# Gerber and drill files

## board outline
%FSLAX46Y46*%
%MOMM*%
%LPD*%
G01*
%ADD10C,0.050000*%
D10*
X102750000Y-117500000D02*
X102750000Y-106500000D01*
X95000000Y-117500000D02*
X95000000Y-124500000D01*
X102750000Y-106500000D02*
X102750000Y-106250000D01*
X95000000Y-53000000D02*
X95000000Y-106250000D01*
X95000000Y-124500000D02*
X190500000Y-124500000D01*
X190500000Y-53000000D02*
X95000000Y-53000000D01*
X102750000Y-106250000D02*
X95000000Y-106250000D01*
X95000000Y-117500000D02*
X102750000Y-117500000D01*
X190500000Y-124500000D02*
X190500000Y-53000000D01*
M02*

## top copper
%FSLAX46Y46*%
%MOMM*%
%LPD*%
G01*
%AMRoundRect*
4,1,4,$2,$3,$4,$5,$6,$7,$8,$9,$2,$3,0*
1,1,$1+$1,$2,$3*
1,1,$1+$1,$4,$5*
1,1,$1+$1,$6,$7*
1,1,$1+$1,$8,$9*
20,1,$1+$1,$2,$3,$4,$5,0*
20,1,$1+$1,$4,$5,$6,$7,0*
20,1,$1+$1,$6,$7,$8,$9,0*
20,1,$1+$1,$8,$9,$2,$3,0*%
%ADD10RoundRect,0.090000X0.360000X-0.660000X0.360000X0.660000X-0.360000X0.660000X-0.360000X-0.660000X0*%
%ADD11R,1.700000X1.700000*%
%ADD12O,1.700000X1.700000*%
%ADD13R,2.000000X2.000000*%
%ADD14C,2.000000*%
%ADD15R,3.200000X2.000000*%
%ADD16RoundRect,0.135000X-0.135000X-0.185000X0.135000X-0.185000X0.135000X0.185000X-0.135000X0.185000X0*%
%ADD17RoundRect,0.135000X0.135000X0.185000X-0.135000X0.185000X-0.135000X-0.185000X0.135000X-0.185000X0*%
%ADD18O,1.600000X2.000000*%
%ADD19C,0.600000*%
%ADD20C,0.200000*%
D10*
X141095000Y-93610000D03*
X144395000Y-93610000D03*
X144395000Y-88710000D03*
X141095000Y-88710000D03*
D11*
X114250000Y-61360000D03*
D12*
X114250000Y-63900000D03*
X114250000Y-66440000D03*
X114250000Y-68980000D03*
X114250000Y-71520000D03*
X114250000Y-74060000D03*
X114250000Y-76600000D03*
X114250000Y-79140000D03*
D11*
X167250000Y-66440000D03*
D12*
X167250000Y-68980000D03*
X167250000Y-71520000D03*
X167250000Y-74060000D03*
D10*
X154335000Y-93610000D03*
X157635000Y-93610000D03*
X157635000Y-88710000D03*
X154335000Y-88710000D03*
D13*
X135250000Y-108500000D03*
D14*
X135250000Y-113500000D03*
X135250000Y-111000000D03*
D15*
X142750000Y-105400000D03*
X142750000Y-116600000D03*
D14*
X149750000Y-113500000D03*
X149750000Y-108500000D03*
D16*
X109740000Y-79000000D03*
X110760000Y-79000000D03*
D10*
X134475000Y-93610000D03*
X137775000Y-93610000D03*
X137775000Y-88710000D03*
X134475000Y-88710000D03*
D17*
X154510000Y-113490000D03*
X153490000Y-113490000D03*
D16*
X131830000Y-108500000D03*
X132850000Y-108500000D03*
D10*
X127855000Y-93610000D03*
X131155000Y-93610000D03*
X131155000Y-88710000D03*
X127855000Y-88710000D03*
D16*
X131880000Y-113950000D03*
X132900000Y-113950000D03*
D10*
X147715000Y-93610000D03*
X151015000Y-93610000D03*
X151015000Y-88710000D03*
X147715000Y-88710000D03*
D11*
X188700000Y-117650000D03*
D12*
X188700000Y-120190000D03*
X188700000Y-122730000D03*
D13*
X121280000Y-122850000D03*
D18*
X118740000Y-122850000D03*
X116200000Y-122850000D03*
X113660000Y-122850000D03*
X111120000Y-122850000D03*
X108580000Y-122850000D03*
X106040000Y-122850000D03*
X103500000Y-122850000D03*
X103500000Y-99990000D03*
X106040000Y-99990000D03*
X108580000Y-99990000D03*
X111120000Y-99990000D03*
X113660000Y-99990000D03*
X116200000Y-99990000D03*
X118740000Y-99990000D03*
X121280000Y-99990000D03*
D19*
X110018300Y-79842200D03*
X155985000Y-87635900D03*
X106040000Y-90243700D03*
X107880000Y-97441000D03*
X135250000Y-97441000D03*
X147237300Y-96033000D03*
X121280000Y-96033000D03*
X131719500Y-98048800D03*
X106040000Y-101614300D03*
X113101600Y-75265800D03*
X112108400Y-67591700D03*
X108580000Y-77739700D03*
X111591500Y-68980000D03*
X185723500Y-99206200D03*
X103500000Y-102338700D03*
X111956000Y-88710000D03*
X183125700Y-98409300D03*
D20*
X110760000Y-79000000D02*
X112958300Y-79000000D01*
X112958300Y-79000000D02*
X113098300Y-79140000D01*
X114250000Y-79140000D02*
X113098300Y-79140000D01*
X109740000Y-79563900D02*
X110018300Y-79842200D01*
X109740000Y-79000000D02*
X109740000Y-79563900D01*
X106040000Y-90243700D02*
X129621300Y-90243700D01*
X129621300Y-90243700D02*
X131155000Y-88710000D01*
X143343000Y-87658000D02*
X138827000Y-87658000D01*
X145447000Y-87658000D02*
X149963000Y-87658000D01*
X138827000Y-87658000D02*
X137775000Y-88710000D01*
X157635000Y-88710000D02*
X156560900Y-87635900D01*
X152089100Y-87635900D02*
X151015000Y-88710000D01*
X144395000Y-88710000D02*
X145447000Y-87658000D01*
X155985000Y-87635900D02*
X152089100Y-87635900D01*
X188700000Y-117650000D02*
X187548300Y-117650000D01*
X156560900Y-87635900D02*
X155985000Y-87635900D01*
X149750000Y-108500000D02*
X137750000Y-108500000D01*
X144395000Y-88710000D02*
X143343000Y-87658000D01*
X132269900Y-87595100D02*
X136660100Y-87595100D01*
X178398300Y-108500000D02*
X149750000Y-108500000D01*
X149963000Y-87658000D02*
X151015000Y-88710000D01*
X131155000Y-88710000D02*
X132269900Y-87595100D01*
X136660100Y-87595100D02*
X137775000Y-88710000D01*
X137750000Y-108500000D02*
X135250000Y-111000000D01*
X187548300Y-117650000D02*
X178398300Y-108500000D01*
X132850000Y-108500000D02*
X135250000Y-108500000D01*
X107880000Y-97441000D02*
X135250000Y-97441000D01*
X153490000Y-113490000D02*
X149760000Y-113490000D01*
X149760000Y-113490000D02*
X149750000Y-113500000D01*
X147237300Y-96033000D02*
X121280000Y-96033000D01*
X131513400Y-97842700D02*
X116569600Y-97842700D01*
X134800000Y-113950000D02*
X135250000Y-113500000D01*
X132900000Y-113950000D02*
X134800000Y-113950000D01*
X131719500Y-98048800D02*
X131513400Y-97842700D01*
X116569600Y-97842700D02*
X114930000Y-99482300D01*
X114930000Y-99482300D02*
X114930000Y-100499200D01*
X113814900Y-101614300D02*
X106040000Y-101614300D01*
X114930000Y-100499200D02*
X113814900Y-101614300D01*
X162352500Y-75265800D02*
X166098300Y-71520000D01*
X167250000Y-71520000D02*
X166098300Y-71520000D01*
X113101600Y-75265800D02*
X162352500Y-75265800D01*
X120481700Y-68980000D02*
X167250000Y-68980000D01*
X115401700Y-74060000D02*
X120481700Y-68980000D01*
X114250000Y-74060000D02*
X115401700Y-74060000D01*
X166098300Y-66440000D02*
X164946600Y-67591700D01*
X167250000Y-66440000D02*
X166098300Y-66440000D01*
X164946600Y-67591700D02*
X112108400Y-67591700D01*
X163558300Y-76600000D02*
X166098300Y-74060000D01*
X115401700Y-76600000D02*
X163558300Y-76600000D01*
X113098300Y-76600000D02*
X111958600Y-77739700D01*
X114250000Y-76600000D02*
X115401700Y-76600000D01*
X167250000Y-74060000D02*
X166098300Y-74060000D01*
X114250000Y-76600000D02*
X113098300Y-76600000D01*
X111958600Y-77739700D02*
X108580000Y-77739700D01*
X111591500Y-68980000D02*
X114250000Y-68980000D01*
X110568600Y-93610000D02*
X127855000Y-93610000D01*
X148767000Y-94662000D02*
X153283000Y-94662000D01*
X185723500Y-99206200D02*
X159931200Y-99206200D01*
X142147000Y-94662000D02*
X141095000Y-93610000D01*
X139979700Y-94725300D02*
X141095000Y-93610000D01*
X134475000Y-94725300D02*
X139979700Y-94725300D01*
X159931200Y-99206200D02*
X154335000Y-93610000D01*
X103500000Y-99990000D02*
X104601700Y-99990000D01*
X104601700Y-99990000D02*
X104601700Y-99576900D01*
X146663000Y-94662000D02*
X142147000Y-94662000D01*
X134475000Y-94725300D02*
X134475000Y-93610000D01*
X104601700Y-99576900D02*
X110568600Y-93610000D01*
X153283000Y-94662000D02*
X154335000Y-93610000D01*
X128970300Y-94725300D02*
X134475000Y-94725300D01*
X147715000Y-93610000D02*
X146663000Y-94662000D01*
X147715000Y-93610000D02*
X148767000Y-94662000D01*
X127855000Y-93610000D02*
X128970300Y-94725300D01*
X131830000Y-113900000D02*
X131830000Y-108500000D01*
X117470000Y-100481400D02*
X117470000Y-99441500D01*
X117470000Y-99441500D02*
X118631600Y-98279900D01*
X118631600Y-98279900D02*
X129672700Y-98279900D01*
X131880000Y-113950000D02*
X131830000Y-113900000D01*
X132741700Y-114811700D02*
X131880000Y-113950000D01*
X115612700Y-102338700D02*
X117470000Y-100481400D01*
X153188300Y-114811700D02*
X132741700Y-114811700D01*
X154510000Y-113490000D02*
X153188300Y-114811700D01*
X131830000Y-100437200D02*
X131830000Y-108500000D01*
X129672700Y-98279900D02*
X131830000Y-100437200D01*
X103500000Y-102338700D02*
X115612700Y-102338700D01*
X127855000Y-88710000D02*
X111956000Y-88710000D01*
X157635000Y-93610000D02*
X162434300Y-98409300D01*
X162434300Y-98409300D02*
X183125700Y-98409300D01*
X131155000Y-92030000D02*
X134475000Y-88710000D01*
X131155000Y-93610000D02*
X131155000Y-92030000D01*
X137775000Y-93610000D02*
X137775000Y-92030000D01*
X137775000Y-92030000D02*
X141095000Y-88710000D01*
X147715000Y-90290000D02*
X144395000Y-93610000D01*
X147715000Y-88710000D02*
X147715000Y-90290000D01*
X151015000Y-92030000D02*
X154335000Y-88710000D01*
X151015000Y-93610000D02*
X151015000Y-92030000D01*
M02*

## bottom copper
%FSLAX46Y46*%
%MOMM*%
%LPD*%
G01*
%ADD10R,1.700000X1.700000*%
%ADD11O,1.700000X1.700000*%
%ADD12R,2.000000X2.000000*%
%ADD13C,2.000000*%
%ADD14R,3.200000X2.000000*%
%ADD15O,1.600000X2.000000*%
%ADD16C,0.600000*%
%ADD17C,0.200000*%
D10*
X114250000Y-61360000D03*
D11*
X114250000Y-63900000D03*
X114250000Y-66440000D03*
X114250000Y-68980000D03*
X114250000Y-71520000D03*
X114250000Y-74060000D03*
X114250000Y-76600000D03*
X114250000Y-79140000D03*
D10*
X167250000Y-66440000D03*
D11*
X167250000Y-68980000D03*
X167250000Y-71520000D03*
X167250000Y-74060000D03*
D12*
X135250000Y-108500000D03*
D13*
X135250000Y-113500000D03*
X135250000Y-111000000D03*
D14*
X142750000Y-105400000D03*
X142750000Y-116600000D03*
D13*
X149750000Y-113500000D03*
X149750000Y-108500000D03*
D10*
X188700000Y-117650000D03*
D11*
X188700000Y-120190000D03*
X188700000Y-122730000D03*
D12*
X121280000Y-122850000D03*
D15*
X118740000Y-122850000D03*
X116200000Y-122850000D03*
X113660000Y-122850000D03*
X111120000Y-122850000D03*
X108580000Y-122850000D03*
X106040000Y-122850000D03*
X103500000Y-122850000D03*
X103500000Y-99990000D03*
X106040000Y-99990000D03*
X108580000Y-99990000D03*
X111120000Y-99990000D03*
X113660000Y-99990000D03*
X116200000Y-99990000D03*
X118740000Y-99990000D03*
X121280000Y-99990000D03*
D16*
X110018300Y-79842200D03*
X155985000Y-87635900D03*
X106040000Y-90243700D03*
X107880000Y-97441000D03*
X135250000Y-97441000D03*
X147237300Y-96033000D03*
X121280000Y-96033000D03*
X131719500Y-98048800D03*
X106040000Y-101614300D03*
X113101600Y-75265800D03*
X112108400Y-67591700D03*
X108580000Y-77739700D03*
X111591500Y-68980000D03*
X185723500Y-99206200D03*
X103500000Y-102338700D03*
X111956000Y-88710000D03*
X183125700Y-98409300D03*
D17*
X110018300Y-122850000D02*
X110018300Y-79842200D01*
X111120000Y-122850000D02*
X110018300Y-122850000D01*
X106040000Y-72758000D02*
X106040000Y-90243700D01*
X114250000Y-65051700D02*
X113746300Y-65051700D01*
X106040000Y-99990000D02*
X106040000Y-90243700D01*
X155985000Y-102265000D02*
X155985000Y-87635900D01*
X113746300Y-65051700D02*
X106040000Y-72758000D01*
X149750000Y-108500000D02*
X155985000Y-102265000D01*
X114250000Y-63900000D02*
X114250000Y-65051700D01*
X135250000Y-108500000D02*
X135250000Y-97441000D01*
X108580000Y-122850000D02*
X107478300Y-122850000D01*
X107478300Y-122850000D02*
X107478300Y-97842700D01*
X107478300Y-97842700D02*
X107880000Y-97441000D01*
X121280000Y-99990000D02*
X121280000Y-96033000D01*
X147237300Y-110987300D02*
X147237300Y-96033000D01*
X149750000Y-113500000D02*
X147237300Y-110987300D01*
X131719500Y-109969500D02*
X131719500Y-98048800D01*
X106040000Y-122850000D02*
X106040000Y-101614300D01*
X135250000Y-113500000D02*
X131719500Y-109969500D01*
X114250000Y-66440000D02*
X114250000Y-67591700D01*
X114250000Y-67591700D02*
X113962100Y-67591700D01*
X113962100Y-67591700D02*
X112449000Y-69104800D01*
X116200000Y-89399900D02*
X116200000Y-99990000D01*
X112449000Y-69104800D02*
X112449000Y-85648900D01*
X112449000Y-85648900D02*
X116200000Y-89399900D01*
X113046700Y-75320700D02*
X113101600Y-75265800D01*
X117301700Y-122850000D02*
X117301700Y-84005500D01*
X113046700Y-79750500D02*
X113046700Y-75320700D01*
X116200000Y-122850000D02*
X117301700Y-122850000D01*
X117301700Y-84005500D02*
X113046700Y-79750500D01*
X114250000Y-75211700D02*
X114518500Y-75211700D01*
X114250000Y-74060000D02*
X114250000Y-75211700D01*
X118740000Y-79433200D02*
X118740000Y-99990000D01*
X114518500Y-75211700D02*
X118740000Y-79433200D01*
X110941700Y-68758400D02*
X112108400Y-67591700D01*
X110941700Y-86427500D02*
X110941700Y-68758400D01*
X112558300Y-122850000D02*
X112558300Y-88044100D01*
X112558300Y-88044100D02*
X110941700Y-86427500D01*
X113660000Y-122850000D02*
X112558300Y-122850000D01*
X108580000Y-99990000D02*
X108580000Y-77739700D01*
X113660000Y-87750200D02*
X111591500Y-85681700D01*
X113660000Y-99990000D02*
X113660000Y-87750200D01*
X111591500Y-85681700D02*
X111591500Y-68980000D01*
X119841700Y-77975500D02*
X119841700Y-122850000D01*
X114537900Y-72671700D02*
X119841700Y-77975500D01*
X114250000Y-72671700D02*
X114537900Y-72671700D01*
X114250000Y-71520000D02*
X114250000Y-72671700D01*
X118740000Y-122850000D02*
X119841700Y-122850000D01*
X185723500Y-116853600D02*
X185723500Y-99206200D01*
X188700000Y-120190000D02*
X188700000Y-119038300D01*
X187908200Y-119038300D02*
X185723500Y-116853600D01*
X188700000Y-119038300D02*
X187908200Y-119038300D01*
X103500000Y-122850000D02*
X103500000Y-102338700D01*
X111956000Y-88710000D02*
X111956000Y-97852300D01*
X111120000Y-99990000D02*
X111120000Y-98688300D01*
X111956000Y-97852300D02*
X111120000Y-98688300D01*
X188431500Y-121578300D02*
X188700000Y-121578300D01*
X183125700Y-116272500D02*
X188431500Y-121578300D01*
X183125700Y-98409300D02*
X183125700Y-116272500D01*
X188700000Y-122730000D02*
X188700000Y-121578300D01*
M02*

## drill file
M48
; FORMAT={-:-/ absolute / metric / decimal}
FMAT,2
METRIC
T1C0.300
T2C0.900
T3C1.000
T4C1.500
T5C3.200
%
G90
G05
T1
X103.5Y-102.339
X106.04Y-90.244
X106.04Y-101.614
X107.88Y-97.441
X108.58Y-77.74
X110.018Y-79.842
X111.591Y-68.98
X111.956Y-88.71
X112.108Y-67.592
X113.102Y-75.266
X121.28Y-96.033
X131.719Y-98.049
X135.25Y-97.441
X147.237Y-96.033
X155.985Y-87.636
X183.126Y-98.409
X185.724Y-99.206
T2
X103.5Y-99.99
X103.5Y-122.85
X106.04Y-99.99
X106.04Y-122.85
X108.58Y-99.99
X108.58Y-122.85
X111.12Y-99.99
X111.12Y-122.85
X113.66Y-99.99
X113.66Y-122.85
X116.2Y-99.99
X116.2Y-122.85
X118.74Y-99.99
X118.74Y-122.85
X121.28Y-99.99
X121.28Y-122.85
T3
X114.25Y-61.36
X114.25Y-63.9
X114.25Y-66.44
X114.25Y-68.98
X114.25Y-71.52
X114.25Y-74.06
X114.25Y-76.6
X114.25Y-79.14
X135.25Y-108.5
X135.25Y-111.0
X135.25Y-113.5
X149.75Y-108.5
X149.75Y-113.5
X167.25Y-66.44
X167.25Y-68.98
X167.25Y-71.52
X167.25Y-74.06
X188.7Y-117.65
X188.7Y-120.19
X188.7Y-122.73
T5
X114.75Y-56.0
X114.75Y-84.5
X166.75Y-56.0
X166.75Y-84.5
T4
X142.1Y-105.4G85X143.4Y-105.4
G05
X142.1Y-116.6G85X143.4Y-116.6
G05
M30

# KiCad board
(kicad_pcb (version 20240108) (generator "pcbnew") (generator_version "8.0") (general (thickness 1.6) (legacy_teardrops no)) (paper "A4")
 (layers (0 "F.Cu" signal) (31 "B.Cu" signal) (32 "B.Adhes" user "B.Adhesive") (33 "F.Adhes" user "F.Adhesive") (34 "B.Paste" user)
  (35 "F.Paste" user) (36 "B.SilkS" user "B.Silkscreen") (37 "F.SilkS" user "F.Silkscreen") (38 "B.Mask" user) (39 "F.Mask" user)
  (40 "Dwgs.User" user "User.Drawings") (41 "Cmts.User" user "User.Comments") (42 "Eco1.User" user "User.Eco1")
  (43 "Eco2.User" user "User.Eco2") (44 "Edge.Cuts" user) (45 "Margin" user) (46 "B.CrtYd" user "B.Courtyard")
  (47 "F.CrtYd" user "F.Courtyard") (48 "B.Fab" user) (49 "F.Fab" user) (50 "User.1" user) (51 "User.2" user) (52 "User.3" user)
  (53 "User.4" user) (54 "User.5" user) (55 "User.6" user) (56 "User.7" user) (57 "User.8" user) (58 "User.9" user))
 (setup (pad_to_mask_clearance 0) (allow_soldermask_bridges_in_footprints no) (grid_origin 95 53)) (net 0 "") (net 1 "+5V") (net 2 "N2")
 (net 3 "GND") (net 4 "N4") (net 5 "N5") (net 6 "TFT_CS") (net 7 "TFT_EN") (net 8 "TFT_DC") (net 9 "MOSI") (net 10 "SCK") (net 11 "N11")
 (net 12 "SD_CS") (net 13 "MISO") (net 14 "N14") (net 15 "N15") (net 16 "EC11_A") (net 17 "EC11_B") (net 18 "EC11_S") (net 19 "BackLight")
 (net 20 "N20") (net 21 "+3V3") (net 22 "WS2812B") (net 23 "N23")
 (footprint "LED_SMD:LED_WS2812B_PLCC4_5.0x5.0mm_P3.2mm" (layer "F.Cu") (at 142.745 91.16 90)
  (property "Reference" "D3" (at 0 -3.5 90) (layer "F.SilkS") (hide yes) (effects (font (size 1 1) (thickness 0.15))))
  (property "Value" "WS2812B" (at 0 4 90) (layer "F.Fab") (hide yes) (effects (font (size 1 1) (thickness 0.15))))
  (pad "1" smd roundrect (at -2.45 -1.65 90) (size 1.5 0.9) (layers "F.Cu" "F.Paste" "F.Mask") (roundrect_rratio 0.1) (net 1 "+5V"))
  (pad "2" smd roundrect (at -2.45 1.65 90) (size 1.5 0.9) (layers "F.Cu" "F.Paste" "F.Mask") (roundrect_rratio 0.1) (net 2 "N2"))
  (pad "3" smd roundrect (at 2.45 1.65 90) (size 1.5 0.9) (layers "F.Cu" "F.Paste" "F.Mask") (roundrect_rratio 0.1) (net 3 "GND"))
  (pad "4" smd roundrect (at 2.45 -1.65 90) (size 1.5 0.9) (layers "F.Cu" "F.Paste" "F.Mask") (roundrect_rratio 0.1) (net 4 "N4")))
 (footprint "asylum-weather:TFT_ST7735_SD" (layer "F.Cu") (at 134.25 70)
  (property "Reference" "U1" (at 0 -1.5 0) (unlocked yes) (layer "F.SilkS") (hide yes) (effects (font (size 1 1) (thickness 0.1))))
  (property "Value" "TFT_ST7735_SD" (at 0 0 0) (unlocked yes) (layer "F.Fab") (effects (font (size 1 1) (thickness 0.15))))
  (pad "" np_thru_hole circle (at -19.5 -14) (size 3.2 3.2) (drill 3.2) (layers "*.Cu" "*.Mask"))
  (pad "" np_thru_hole circle (at -19.5 14.5) (size 3.2 3.2) (drill 3.2) (layers "*.Cu" "*.Mask"))
  (pad "" np_thru_hole circle (at 32.5 -14) (size 3.2 3.2) (drill 3.2) (layers "*.Cu" "*.Mask"))
  (pad "" np_thru_hole circle (at 32.5 14.5) (size 3.2 3.2) (drill 3.2) (layers "*.Cu" "*.Mask"))
  (pad "1" thru_hole rect (at -20 -8.64) (size 1.7 1.7) (drill 1) (layers "*.Cu" "*.Mask") (remove_unused_layers no) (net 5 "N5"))
  (pad "2" thru_hole oval (at -20 -6.1) (size 1.7 1.7) (drill 1) (layers "*.Cu" "*.Mask") (remove_unused_layers no) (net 3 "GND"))
  (pad "3" thru_hole oval (at -20 -3.56) (size 1.7 1.7) (drill 1) (layers "*.Cu" "*.Mask") (remove_unused_layers no) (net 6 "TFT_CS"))
  (pad "4" thru_hole oval (at -20 -1.02) (size 1.7 1.7) (drill 1) (layers "*.Cu" "*.Mask") (remove_unused_layers no) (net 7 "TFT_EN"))
  (pad "5" thru_hole oval (at -20 1.52) (size 1.7 1.7) (drill 1) (layers "*.Cu" "*.Mask") (remove_unused_layers no) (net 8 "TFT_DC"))
  (pad "6" thru_hole oval (at -20 4.06) (size 1.7 1.7) (drill 1) (layers "*.Cu" "*.Mask") (remove_unused_layers no) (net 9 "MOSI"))
  (pad "7" thru_hole oval (at -20 6.6) (size 1.7 1.7) (drill 1) (layers "*.Cu" "*.Mask") (remove_unused_layers no) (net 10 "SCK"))
  (pad "8" thru_hole oval (at -20 9.14) (size 1.7 1.7) (drill 1) (layers "*.Cu" "*.Mask") (remove_unused_layers no) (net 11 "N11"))
  (pad "9" thru_hole rect (at 33 -3.56) (size 1.7 1.7) (drill 1) (layers "*.Cu" "*.Mask") (remove_unused_layers no) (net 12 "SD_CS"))
  (pad "10" thru_hole oval (at 33 -1.02) (size 1.7 1.7) (drill 1) (layers "*.Cu" "*.Mask") (remove_unused_layers no) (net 9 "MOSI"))
  (pad "11" thru_hole oval (at 33 1.52) (size 1.7 1.7) (drill 1) (layers "*.Cu" "*.Mask") (remove_unused_layers no) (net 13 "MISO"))
  (pad "12" thru_hole oval (at 33 4.06) (size 1.7 1.7) (drill 1) (layers "*.Cu" "*.Mask") (remove_unused_layers no) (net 10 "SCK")))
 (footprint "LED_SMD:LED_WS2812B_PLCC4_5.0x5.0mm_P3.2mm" (layer "F.Cu") (at 155.985 91.16 90)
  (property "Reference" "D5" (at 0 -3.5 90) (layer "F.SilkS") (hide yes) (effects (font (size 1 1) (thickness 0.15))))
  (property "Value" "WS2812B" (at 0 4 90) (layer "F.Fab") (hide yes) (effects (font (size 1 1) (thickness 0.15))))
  (pad "1" smd roundrect (at -2.45 -1.65 90) (size 1.5 0.9) (layers "F.Cu" "F.Paste" "F.Mask") (roundrect_rratio 0.1) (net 1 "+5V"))
  (pad "2" smd roundrect (at -2.45 1.65 90) (size 1.5 0.9) (layers "F.Cu" "F.Paste" "F.Mask") (roundrect_rratio 0.1) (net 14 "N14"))
  (pad "3" smd roundrect (at 2.45 1.65 90) (size 1.5 0.9) (layers "F.Cu" "F.Paste" "F.Mask") (roundrect_rratio 0.1) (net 3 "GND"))
  (pad "4" smd roundrect (at 2.45 -1.65 90) (size 1.5 0.9) (layers "F.Cu" "F.Paste" "F.Mask") (roundrect_rratio 0.1) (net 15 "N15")))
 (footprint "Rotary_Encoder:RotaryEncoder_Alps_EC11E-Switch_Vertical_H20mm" (layer "F.Cu") (at 135.25 108.5)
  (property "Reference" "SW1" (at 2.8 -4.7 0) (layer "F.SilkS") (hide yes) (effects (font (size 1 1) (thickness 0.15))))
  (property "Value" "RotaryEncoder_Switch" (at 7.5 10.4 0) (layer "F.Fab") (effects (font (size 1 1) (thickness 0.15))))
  (pad "A" thru_hole rect (at 0 0) (size 2 2) (drill 1) (layers "*.Cu" "*.Mask") (remove_unused_layers no) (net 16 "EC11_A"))
  (pad "B" thru_hole circle (at 0 5) (size 2 2) (drill 1) (layers "*.Cu" "*.Mask") (remove_unused_layers no) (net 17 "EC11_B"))
  (pad "C" thru_hole circle (at 0 2.5) (size 2 2) (drill 1) (layers "*.Cu" "*.Mask") (remove_unused_layers no) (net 3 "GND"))
  (pad "MP" thru_hole rect (at 7.5 -3.1) (size 3.2 2) (drill oval 2.8 1.5) (layers "*.Cu" "*.Mask") (remove_unused_layers no))
  (pad "MP" thru_hole rect (at 7.5 8.1) (size 3.2 2) (drill oval 2.8 1.5) (layers "*.Cu" "*.Mask") (remove_unused_layers no))
  (pad "S1" thru_hole circle (at 14.5 5) (size 2 2) (drill 1) (layers "*.Cu" "*.Mask") (remove_unused_layers no) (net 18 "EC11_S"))
  (pad "S2" thru_hole circle (at 14.5 0) (size 2 2) (drill 1) (layers "*.Cu" "*.Mask") (remove_unused_layers no) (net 3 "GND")))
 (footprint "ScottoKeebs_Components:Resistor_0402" (layer "F.Cu") (at 110.25 79)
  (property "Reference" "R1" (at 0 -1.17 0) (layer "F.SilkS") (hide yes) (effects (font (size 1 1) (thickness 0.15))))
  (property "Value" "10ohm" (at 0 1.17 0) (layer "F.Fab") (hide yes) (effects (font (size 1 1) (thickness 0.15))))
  (pad "1" smd roundrect (at -0.51 0) (size 0.54 0.64) (layers "F.Cu" "F.Paste" "F.Mask") (roundrect_rratio 0.25) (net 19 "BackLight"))
  (pad "2" smd roundrect (at 0.51 0) (size 0.54 0.64) (layers "F.Cu" "F.Paste" "F.Mask") (roundrect_rratio 0.25) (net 11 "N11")))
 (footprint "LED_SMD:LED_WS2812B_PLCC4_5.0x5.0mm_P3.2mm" (layer "F.Cu") (at 136.125 91.16 90)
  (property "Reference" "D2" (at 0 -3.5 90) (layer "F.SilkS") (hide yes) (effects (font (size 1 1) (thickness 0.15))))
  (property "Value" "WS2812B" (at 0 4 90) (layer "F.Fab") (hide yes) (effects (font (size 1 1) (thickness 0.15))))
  (pad "1" smd roundrect (at -2.45 -1.65 90) (size 1.5 0.9) (layers "F.Cu" "F.Paste" "F.Mask") (roundrect_rratio 0.1) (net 1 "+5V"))
  (pad "2" smd roundrect (at -2.45 1.65 90) (size 1.5 0.9) (layers "F.Cu" "F.Paste" "F.Mask") (roundrect_rratio 0.1) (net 4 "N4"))
  (pad "3" smd roundrect (at 2.45 1.65 90) (size 1.5 0.9) (layers "F.Cu" "F.Paste" "F.Mask") (roundrect_rratio 0.1) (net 3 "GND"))
  (pad "4" smd roundrect (at 2.45 -1.65 90) (size 1.5 0.9) (layers "F.Cu" "F.Paste" "F.Mask") (roundrect_rratio 0.1) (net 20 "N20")))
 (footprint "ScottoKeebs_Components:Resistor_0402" (layer "F.Cu") (at 154 113.49 180)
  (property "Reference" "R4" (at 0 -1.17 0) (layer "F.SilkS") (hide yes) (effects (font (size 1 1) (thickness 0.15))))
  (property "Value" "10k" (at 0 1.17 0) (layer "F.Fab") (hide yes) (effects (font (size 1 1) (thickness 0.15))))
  (pad "1" smd roundrect (at -0.51 0 180) (size 0.54 0.64) (layers "F.Cu" "F.Paste" "F.Mask") (roundrect_rratio 0.25) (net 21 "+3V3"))
  (pad "2" smd roundrect (at 0.51 0 180) (size 0.54 0.64) (layers "F.Cu" "F.Paste" "F.Mask") (roundrect_rratio 0.25) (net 18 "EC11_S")))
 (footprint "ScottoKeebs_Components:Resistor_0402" (layer "F.Cu") (at 132.34 108.5)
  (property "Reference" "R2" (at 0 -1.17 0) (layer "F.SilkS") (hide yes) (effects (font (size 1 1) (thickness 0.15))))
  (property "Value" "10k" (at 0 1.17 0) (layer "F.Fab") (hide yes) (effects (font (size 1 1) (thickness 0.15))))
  (pad "1" smd roundrect (at -0.51 0) (size 0.54 0.64) (layers "F.Cu" "F.Paste" "F.Mask") (roundrect_rratio 0.25) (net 21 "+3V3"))
  (pad "2" smd roundrect (at 0.51 0) (size 0.54 0.64) (layers "F.Cu" "F.Paste" "F.Mask") (roundrect_rratio 0.25) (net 16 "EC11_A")))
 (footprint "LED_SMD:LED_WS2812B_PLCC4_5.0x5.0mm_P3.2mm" (layer "F.Cu") (at 129.505 91.16 90)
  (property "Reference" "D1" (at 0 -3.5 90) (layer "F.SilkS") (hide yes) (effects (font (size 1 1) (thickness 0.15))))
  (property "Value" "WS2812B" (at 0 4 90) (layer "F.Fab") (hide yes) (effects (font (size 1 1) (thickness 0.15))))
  (pad "1" smd roundrect (at -2.45 -1.65 90) (size 1.5 0.9) (layers "F.Cu" "F.Paste" "F.Mask") (roundrect_rratio 0.1) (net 1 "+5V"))
  (pad "2" smd roundrect (at -2.45 1.65 90) (size 1.5 0.9) (layers "F.Cu" "F.Paste" "F.Mask") (roundrect_rratio 0.1) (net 20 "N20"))
  (pad "3" smd roundrect (at 2.45 1.65 90) (size 1.5 0.9) (layers "F.Cu" "F.Paste" "F.Mask") (roundrect_rratio 0.1) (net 3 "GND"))
  (pad "4" smd roundrect (at 2.45 -1.65 90) (size 1.5 0.9) (layers "F.Cu" "F.Paste" "F.Mask") (roundrect_rratio 0.1) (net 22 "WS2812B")))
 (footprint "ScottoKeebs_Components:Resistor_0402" (layer "F.Cu") (at 132.39 113.95)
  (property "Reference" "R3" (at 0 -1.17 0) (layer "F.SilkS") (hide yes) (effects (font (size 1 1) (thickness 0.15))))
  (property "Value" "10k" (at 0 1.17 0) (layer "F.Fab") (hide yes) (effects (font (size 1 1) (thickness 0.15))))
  (pad "1" smd roundrect (at -0.51 0) (size 0.54 0.64) (layers "F.Cu" "F.Paste" "F.Mask") (roundrect_rratio 0.25) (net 21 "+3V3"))
  (pad "2" smd roundrect (at 0.51 0) (size 0.54 0.64) (layers "F.Cu" "F.Paste" "F.Mask") (roundrect_rratio 0.25) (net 17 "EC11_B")))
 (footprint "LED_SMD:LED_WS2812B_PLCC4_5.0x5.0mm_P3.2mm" (layer "F.Cu") (at 149.365 91.16 90)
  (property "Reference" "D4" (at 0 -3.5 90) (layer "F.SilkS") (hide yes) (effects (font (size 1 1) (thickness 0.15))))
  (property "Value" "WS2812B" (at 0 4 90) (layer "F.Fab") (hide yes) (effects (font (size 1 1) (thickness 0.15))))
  (pad "1" smd roundrect (at -2.45 -1.65 90) (size 1.5 0.9) (layers "F.Cu" "F.Paste" "F.Mask") (roundrect_rratio 0.1) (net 1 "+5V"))
  (pad "2" smd roundrect (at -2.45 1.65 90) (size 1.5 0.9) (layers "F.Cu" "F.Paste" "F.Mask") (roundrect_rratio 0.1) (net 15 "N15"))
  (pad "3" smd roundrect (at 2.45 1.65 90) (size 1.5 0.9) (layers "F.Cu" "F.Paste" "F.Mask") (roundrect_rratio 0.1) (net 3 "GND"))
  (pad "4" smd roundrect (at 2.45 -1.65 90) (size 1.5 0.9) (layers "F.Cu" "F.Paste" "F.Mask") (roundrect_rratio 0.1) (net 2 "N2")))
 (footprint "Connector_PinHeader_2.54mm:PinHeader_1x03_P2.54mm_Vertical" (layer "B.Cu") (at 188.7 117.65 180)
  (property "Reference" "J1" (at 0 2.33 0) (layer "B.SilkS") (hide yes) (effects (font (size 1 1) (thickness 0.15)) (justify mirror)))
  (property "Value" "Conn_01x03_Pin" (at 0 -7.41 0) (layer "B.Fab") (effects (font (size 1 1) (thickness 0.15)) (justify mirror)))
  (pad "1" thru_hole rect (at 0 0 180) (size 1.7 1.7) (drill 1) (layers "*.Cu" "*.Mask") (remove_unused_layers no) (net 3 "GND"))
  (pad "2" thru_hole oval (at 0 -2.54 180) (size 1.7 1.7) (drill 1) (layers "*.Cu" "*.Mask") (remove_unused_layers no) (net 1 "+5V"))
  (pad "3" thru_hole oval (at 0 -5.08 180) (size 1.7 1.7) (drill 1) (layers "*.Cu" "*.Mask") (remove_unused_layers no) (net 14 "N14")))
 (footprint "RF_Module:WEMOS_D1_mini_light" (layer "B.Cu") (at 121.28 122.85 90)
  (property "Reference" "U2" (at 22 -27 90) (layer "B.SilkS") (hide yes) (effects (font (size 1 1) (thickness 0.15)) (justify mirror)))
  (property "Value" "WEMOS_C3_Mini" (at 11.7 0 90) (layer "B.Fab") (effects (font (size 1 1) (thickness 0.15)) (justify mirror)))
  (pad "1" thru_hole rect (at 0 0 90) (size 2 2) (drill 0.9) (layers "*.Cu" "*.Mask") (remove_unused_layers no) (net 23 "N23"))
  (pad "2" thru_hole oval (at 0 -2.54 90) (size 2 1.6) (drill 0.9) (layers "*.Cu" "*.Mask") (remove_unused_layers no) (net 8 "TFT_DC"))
  (pad "3" thru_hole oval (at 0 -5.08 90) (size 2 1.6) (drill 0.9) (layers "*.Cu" "*.Mask") (remove_unused_layers no) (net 13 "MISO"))
  (pad "4" thru_hole oval (at 0 -7.62 90) (size 2 1.6) (drill 0.9) (layers "*.Cu" "*.Mask") (remove_unused_layers no) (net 12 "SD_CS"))
  (pad "5" thru_hole oval (at 0 -10.16 90) (size 2 1.6) (drill 0.9) (layers "*.Cu" "*.Mask") (remove_unused_layers no) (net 19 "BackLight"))
  (pad "6" thru_hole oval (at 0 -12.7 90) (size 2 1.6) (drill 0.9) (layers "*.Cu" "*.Mask") (remove_unused_layers no) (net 16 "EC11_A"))
  (pad "7" thru_hole oval (at 0 -15.24 90) (size 2 1.6) (drill 0.9) (layers "*.Cu" "*.Mask") (remove_unused_layers no) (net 17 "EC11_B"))
  (pad "8" thru_hole oval (at 0 -17.78 90) (size 2 1.6) (drill 0.9) (layers "*.Cu" "*.Mask") (remove_unused_layers no) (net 21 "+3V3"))
  (pad "9" thru_hole oval (at 22.86 -17.78 90) (size 2 1.6) (drill 0.9) (layers "*.Cu" "*.Mask") (remove_unused_layers no) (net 1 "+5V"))
  (pad "10" thru_hole oval (at 22.86 -15.24 90) (size 2 1.6) (drill 0.9) (layers "*.Cu" "*.Mask") (remove_unused_layers no) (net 3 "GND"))
  (pad "11" thru_hole oval (at 22.86 -12.7 90) (size 2 1.6) (drill 0.9) (layers "*.Cu" "*.Mask") (remove_unused_layers no) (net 10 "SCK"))
  (pad "12" thru_hole oval (at 22.86 -10.16 90) (size 2 1.6) (drill 0.9) (layers "*.Cu" "*.Mask") (remove_unused_layers no)
   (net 22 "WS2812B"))
  (pad "13" thru_hole oval (at 22.86 -7.62 90) (size 2 1.6) (drill 0.9) (layers "*.Cu" "*.Mask") (remove_unused_layers no) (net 7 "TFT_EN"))
  (pad "14" thru_hole oval (at 22.86 -5.08 90) (size 2 1.6) (drill 0.9) (layers "*.Cu" "*.Mask") (remove_unused_layers no) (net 6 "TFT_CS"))
  (pad "15" thru_hole oval (at 22.86 -2.54 90) (size 2 1.6) (drill 0.9) (layers "*.Cu" "*.Mask") (remove_unused_layers no) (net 9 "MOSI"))
  (pad "16" thru_hole oval (at 22.86 0 90) (size 2 1.6) (drill 0.9) (layers "*.Cu" "*.Mask") (remove_unused_layers no) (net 18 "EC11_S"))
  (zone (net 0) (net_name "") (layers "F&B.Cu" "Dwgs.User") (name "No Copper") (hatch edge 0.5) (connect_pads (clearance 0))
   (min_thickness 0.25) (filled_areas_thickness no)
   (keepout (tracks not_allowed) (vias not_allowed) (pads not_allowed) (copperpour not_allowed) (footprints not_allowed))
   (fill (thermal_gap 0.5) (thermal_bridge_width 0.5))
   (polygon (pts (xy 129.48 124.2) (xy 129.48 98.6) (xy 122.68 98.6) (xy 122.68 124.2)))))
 (gr_line (start 102.75 117.5) (end 102.75 106.5) (stroke (width 0.05) (type default)) (layer "Edge.Cuts"))
 (gr_line (start 95 117.5) (end 95 124.5) (stroke (width 0.05) (type default)) (layer "Edge.Cuts"))
 (gr_line (start 102.75 106.5) (end 102.75 106.25) (stroke (width 0.05) (type default)) (layer "Edge.Cuts"))
 (gr_line (start 95 53) (end 95 106.25) (stroke (width 0.05) (type default)) (layer "Edge.Cuts"))
 (gr_line (start 95 124.5) (end 190.5 124.5) (stroke (width 0.05) (type default)) (layer "Edge.Cuts"))
 (gr_line (start 190.5 53) (end 95 53) (stroke (width 0.05) (type default)) (layer "Edge.Cuts"))
 (gr_line (start 102.75 106.25) (end 95 106.25) (stroke (width 0.05) (type default)) (layer "Edge.Cuts"))
 (gr_line (start 95 117.5) (end 102.75 117.5) (stroke (width 0.05) (type default)) (layer "Edge.Cuts"))
 (gr_line (start 190.5 124.5) (end 190.5 53) (stroke (width 0.05) (type default)) (layer "Edge.Cuts"))
 (segment (start 110.76 79) (end 112.9583 79) (width 0.2) (layer "F.Cu") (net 11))
 (segment (start 112.9583 79) (end 113.0983 79.14) (width 0.2) (layer "F.Cu") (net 11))
 (segment (start 114.25 79.14) (end 113.0983 79.14) (width 0.2) (layer "F.Cu") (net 11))
 (segment (start 109.74 79.5639) (end 110.0183 79.8422) (width 0.2) (layer "F.Cu") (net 19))
 (segment (start 109.74 79) (end 109.74 79.5639) (width 0.2) (layer "F.Cu") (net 19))
 (via (at 110.0183 79.8422) (size 0.6) (drill 0.3) (layers "F.Cu" "B.Cu") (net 19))
 (segment (start 110.0183 122.85) (end 110.0183 79.8422) (width 0.2) (layer "B.Cu") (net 19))
 (segment (start 111.12 122.85) (end 110.0183 122.85) (width 0.2) (layer "B.Cu") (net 19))
 (segment (start 106.04 90.2437) (end 129.6213 90.2437) (width 0.2) (layer "F.Cu") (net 3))
 (segment (start 129.6213 90.2437) (end 131.155 88.71) (width 0.2) (layer "F.Cu") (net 3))
 (segment (start 143.343 87.658) (end 138.827 87.658) (width 0.2) (layer "F.Cu") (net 3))
 (segment (start 145.447 87.658) (end 149.963 87.658) (width 0.2) (layer "F.Cu") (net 3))
 (segment (start 138.827 87.658) (end 137.775 88.71) (width 0.2) (layer "F.Cu") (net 3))
 (segment (start 157.635 88.71) (end 156.5609 87.6359) (width 0.2) (layer "F.Cu") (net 3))
 (segment (start 152.0891 87.6359) (end 151.015 88.71) (width 0.2) (layer "F.Cu") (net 3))
 (segment (start 144.395 88.71) (end 145.447 87.658) (width 0.2) (layer "F.Cu") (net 3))
 (segment (start 155.985 87.6359) (end 152.0891 87.6359) (width 0.2) (layer "F.Cu") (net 3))
 (segment (start 188.7 117.65) (end 187.5483 117.65) (width 0.2) (layer "F.Cu") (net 3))
 (segment (start 156.5609 87.6359) (end 155.985 87.6359) (width 0.2) (layer "F.Cu") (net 3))
 (segment (start 149.75 108.5) (end 137.75 108.5) (width 0.2) (layer "F.Cu") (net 3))
 (segment (start 144.395 88.71) (end 143.343 87.658) (width 0.2) (layer "F.Cu") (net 3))
 (segment (start 132.2699 87.5951) (end 136.6601 87.5951) (width 0.2) (layer "F.Cu") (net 3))
 (segment (start 178.3983 108.5) (end 149.75 108.5) (width 0.2) (layer "F.Cu") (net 3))
 (segment (start 149.963 87.658) (end 151.015 88.71) (width 0.2) (layer "F.Cu") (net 3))
 (segment (start 131.155 88.71) (end 132.2699 87.5951) (width 0.2) (layer "F.Cu") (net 3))
 (segment (start 136.6601 87.5951) (end 137.775 88.71) (width 0.2) (layer "F.Cu") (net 3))
 (segment (start 137.75 108.5) (end 135.25 111) (width 0.2) (layer "F.Cu") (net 3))
 (segment (start 187.5483 117.65) (end 178.3983 108.5) (width 0.2) (layer "F.Cu") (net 3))
 (via (at 155.985 87.6359) (size 0.6) (drill 0.3) (layers "F.Cu" "B.Cu") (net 3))
 (via (at 106.04 90.2437) (size 0.6) (drill 0.3) (layers "F.Cu" "B.Cu") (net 3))
 (segment (start 106.04 72.758) (end 106.04 90.2437) (width 0.2) (layer "B.Cu") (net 3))
 (segment (start 114.25 65.0517) (end 113.7463 65.0517) (width 0.2) (layer "B.Cu") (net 3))
 (segment (start 106.04 99.99) (end 106.04 90.2437) (width 0.2) (layer "B.Cu") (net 3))
 (segment (start 155.985 102.265) (end 155.985 87.6359) (width 0.2) (layer "B.Cu") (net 3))
 (segment (start 113.7463 65.0517) (end 106.04 72.758) (width 0.2) (layer "B.Cu") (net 3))
 (segment (start 149.75 108.5) (end 155.985 102.265) (width 0.2) (layer "B.Cu") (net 3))
 (segment (start 114.25 63.9) (end 114.25 65.0517) (width 0.2) (layer "B.Cu") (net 3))
 (segment (start 132.85 108.5) (end 135.25 108.5) (width 0.2) (layer "F.Cu") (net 16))
 (segment (start 107.88 97.441) (end 135.25 97.441) (width 0.2) (layer "F.Cu") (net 16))
 (via (at 107.88 97.441) (size 0.6) (drill 0.3) (layers "F.Cu" "B.Cu") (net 16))
 (via (at 135.25 97.441) (size 0.6) (drill 0.3) (layers "F.Cu" "B.Cu") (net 16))
 (segment (start 135.25 108.5) (end 135.25 97.441) (width 0.2) (layer "B.Cu") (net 16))
 (segment (start 108.58 122.85) (end 107.4783 122.85) (width 0.2) (layer "B.Cu") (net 16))
 (segment (start 107.4783 122.85) (end 107.4783 97.8427) (width 0.2) (layer "B.Cu") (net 16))
 (segment (start 107.4783 97.8427) (end 107.88 97.441) (width 0.2) (layer "B.Cu") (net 16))
 (segment (start 153.49 113.49) (end 149.76 113.49) (width 0.2) (layer "F.Cu") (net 18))
 (segment (start 149.76 113.49) (end 149.75 113.5) (width 0.2) (layer "F.Cu") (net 18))
 (segment (start 147.2373 96.033) (end 121.28 96.033) (width 0.2) (layer "F.Cu") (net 18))
 (via (at 147.2373 96.033) (size 0.6) (drill 0.3) (layers "F.Cu" "B.Cu") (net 18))
 (via (at 121.28 96.033) (size 0.6) (drill 0.3) (layers "F.Cu" "B.Cu") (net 18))
 (segment (start 121.28 99.99) (end 121.28 96.033) (width 0.2) (layer "B.Cu") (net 18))
 (segment (start 147.2373 110.9873) (end 147.2373 96.033) (width 0.2) (layer "B.Cu") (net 18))
 (segment (start 149.75 113.5) (end 147.2373 110.9873) (width 0.2) (layer "B.Cu") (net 18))
 (segment (start 131.5134 97.8427) (end 116.5696 97.8427) (width 0.2) (layer "F.Cu") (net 17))
 (segment (start 134.8 113.95) (end 135.25 113.5) (width 0.2) (layer "F.Cu") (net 17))
 (segment (start 132.9 113.95) (end 134.8 113.95) (width 0.2) (layer "F.Cu") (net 17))
 (segment (start 131.7195 98.0488) (end 131.5134 97.8427) (width 0.2) (layer "F.Cu") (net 17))
 (segment (start 116.5696 97.8427) (end 114.93 99.4823) (width 0.2) (layer "F.Cu") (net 17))
 (segment (start 114.93 99.4823) (end 114.93 100.4992) (width 0.2) (layer "F.Cu") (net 17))
 (segment (start 113.8149 101.6143) (end 106.04 101.6143) (width 0.2) (layer "F.Cu") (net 17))
 (segment (start 114.93 100.4992) (end 113.8149 101.6143) (width 0.2) (layer "F.Cu") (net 17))
 (via (at 131.7195 98.0488) (size 0.6) (drill 0.3) (layers "F.Cu" "B.Cu") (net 17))
 (via (at 106.04 101.6143) (size 0.6) (drill 0.3) (layers "F.Cu" "B.Cu") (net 17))
 (segment (start 131.7195 109.9695) (end 131.7195 98.0488) (width 0.2) (layer "B.Cu") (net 17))
 (segment (start 106.04 122.85) (end 106.04 101.6143) (width 0.2) (layer "B.Cu") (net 17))
 (segment (start 135.25 113.5) (end 131.7195 109.9695) (width 0.2) (layer "B.Cu") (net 17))
 (segment (start 114.25 66.44) (end 114.25 67.5917) (width 0.2) (layer "B.Cu") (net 6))
 (segment (start 114.25 67.5917) (end 113.9621 67.5917) (width 0.2) (layer "B.Cu") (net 6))
 (segment (start 113.9621 67.5917) (end 112.449 69.1048) (width 0.2) (layer "B.Cu") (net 6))
 (segment (start 116.2 89.3999) (end 116.2 99.99) (width 0.2) (layer "B.Cu") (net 6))
 (segment (start 112.449 69.1048) (end 112.449 85.6489) (width 0.2) (layer "B.Cu") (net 6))
 (segment (start 112.449 85.6489) (end 116.2 89.3999) (width 0.2) (layer "B.Cu") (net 6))
 (segment (start 162.3525 75.2658) (end 166.0983 71.52) (width 0.2) (layer "F.Cu") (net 13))
 (segment (start 167.25 71.52) (end 166.0983 71.52) (width 0.2) (layer "F.Cu") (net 13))
 (segment (start 113.1016 75.2658) (end 162.3525 75.2658) (width 0.2) (layer "F.Cu") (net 13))
 (via (at 113.1016 75.2658) (size 0.6) (drill 0.3) (layers "F.Cu" "B.Cu") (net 13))
 (segment (start 113.0467 75.3207) (end 113.1016 75.2658) (width 0.2) (layer "B.Cu") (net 13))
 (segment (start 117.3017 122.85) (end 117.3017 84.0055) (width 0.2) (layer "B.Cu") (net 13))
 (segment (start 113.0467 79.7505) (end 113.0467 75.3207) (width 0.2) (layer "B.Cu") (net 13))
 (segment (start 116.2 122.85) (end 117.3017 122.85) (width 0.2) (layer "B.Cu") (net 13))
 (segment (start 117.3017 84.0055) (end 113.0467 79.7505) (width 0.2) (layer "B.Cu") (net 13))
 (segment (start 120.4817 68.98) (end 167.25 68.98) (width 0.2) (layer "F.Cu") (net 9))
 (segment (start 115.4017 74.06) (end 120.4817 68.98) (width 0.2) (layer "F.Cu") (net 9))
 (segment (start 114.25 74.06) (end 115.4017 74.06) (width 0.2) (layer "F.Cu") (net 9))
 (segment (start 114.25 75.2117) (end 114.5185 75.2117) (width 0.2) (layer "B.Cu") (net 9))
 (segment (start 114.25 74.06) (end 114.25 75.2117) (width 0.2) (layer "B.Cu") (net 9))
 (segment (start 118.74 79.4332) (end 118.74 99.99) (width 0.2) (layer "B.Cu") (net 9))
 (segment (start 114.5185 75.2117) (end 118.74 79.4332) (width 0.2) (layer "B.Cu") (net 9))
 (segment (start 166.0983 66.44) (end 164.9466 67.5917) (width 0.2) (layer "F.Cu") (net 12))
 (segment (start 167.25 66.44) (end 166.0983 66.44) (width 0.2) (layer "F.Cu") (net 12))
 (segment (start 164.9466 67.5917) (end 112.1084 67.5917) (width 0.2) (layer "F.Cu") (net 12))
 (via (at 112.1084 67.5917) (size 0.6) (drill 0.3) (layers "F.Cu" "B.Cu") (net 12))
 (segment (start 110.9417 68.7584) (end 112.1084 67.5917) (width 0.2) (layer "B.Cu") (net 12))
 (segment (start 110.9417 86.4275) (end 110.9417 68.7584) (width 0.2) (layer "B.Cu") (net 12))
 (segment (start 112.5583 122.85) (end 112.5583 88.0441) (width 0.2) (layer "B.Cu") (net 12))
 (segment (start 112.5583 88.0441) (end 110.9417 86.4275) (width 0.2) (layer "B.Cu") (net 12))
 (segment (start 113.66 122.85) (end 112.5583 122.85) (width 0.2) (layer "B.Cu") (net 12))
 (segment (start 163.5583 76.6) (end 166.0983 74.06) (width 0.2) (layer "F.Cu") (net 10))
 (segment (start 115.4017 76.6) (end 163.5583 76.6) (width 0.2) (layer "F.Cu") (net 10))
 (segment (start 113.0983 76.6) (end 111.9586 77.7397) (width 0.2) (layer "F.Cu") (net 10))
 (segment (start 114.25 76.6) (end 115.4017 76.6) (width 0.2) (layer "F.Cu") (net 10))
 (segment (start 167.25 74.06) (end 166.0983 74.06) (width 0.2) (layer "F.Cu") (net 10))
 (segment (start 114.25 76.6) (end 113.0983 76.6) (width 0.2) (layer "F.Cu") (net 10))
 (segment (start 111.9586 77.7397) (end 108.58 77.7397) (width 0.2) (layer "F.Cu") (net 10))
 (via (at 108.58 77.7397) (size 0.6) (drill 0.3) (layers "F.Cu" "B.Cu") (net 10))
 (segment (start 108.58 99.99) (end 108.58 77.7397) (width 0.2) (layer "B.Cu") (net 10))
 (segment (start 111.5915 68.98) (end 114.25 68.98) (width 0.2) (layer "F.Cu") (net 7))
 (via (at 111.5915 68.98) (size 0.6) (drill 0.3) (layers "F.Cu" "B.Cu") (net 7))
 (segment (start 113.66 87.7502) (end 111.5915 85.6817) (width 0.2) (layer "B.Cu") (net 7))
 (segment (start 113.66 99.99) (end 113.66 87.7502) (width 0.2) (layer "B.Cu") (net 7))
 (segment (start 111.5915 85.6817) (end 111.5915 68.98) (width 0.2) (layer "B.Cu") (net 7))
 (segment (start 119.8417 77.9755) (end 119.8417 122.85) (width 0.2) (layer "B.Cu") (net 8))
 (segment (start 114.5379 72.6717) (end 119.8417 77.9755) (width 0.2) (layer "B.Cu") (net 8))
 (segment (start 114.25 72.6717) (end 114.5379 72.6717) (width 0.2) (layer "B.Cu") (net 8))
 (segment (start 114.25 71.52) (end 114.25 72.6717) (width 0.2) (layer "B.Cu") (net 8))
 (segment (start 118.74 122.85) (end 119.8417 122.85) (width 0.2) (layer "B.Cu") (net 8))
 (segment (start 110.5686 93.61) (end 127.855 93.61) (width 0.2) (layer "F.Cu") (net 1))
 (segment (start 148.767 94.662) (end 153.283 94.662) (width 0.2) (layer "F.Cu") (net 1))
 (segment (start 185.7235 99.2062) (end 159.9312 99.2062) (width 0.2) (layer "F.Cu") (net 1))
 (segment (start 142.147 94.662) (end 141.095 93.61) (width 0.2) (layer "F.Cu") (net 1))
 (segment (start 139.9797 94.7253) (end 141.095 93.61) (width 0.2) (layer "F.Cu") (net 1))
 (segment (start 134.475 94.7253) (end 139.9797 94.7253) (width 0.2) (layer "F.Cu") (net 1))
 (segment (start 159.9312 99.2062) (end 154.335 93.61) (width 0.2) (layer "F.Cu") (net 1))
 (segment (start 103.5 99.99) (end 104.6017 99.99) (width 0.2) (layer "F.Cu") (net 1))
 (segment (start 104.6017 99.99) (end 104.6017 99.5769) (width 0.2) (layer "F.Cu") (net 1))
 (segment (start 146.663 94.662) (end 142.147 94.662) (width 0.2) (layer "F.Cu") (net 1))
 (segment (start 134.475 94.7253) (end 134.475 93.61) (width 0.2) (layer "F.Cu") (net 1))
 (segment (start 104.6017 99.5769) (end 110.5686 93.61) (width 0.2) (layer "F.Cu") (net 1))
 (segment (start 153.283 94.662) (end 154.335 93.61) (width 0.2) (layer "F.Cu") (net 1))
 (segment (start 128.9703 94.7253) (end 134.475 94.7253) (width 0.2) (layer "F.Cu") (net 1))
 (segment (start 147.715 93.61) (end 146.663 94.662) (width 0.2) (layer "F.Cu") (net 1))
 (segment (start 147.715 93.61) (end 148.767 94.662) (width 0.2) (layer "F.Cu") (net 1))
 (segment (start 127.855 93.61) (end 128.9703 94.7253) (width 0.2) (layer "F.Cu") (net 1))
 (via (at 185.7235 99.2062) (size 0.6) (drill 0.3) (layers "F.Cu" "B.Cu") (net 1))
 (segment (start 185.7235 116.8536) (end 185.7235 99.2062) (width 0.2) (layer "B.Cu") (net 1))
 (segment (start 188.7 120.19) (end 188.7 119.0383) (width 0.2) (layer "B.Cu") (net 1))
 (segment (start 187.9082 119.0383) (end 185.7235 116.8536) (width 0.2) (layer "B.Cu") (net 1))
 (segment (start 188.7 119.0383) (end 187.9082 119.0383) (width 0.2) (layer "B.Cu") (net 1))
 (segment (start 131.83 113.9) (end 131.83 108.5) (width 0.2) (layer "F.Cu") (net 21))
 (segment (start 117.47 100.4814) (end 117.47 99.4415) (width 0.2) (layer "F.Cu") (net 21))
 (segment (start 117.47 99.4415) (end 118.6316 98.2799) (width 0.2) (layer "F.Cu") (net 21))
 (segment (start 118.6316 98.2799) (end 129.6727 98.2799) (width 0.2) (layer "F.Cu") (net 21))
 (segment (start 131.88 113.95) (end 131.83 113.9) (width 0.2) (layer "F.Cu") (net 21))
 (segment (start 132.7417 114.8117) (end 131.88 113.95) (width 0.2) (layer "F.Cu") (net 21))
 (segment (start 115.6127 102.3387) (end 117.47 100.4814) (width 0.2) (layer "F.Cu") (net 21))
 (segment (start 153.1883 114.8117) (end 132.7417 114.8117) (width 0.2) (layer "F.Cu") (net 21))
 (segment (start 154.51 113.49) (end 153.1883 114.8117) (width 0.2) (layer "F.Cu") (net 21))
 (segment (start 131.83 100.4372) (end 131.83 108.5) (width 0.2) (layer "F.Cu") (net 21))
 (segment (start 129.6727 98.2799) (end 131.83 100.4372) (width 0.2) (layer "F.Cu") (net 21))
 (segment (start 103.5 102.3387) (end 115.6127 102.3387) (width 0.2) (layer "F.Cu") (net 21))
 (via (at 103.5 102.3387) (size 0.6) (drill 0.3) (layers "F.Cu" "B.Cu") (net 21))
 (segment (start 103.5 122.85) (end 103.5 102.3387) (width 0.2) (layer "B.Cu") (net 21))
 (segment (start 127.855 88.71) (end 111.956 88.71) (width 0.2) (layer "F.Cu") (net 22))
 (via (at 111.956 88.71) (size 0.6) (drill 0.3) (layers "F.Cu" "B.Cu") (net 22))
 (segment (start 111.956 88.71) (end 111.956 97.8523) (width 0.2) (layer "B.Cu") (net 22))
 (segment (start 111.12 99.99) (end 111.12 98.6883) (width 0.2) (layer "B.Cu") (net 22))
 (segment (start 111.956 97.8523) (end 111.12 98.6883) (width 0.2) (layer "B.Cu") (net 22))
 (segment (start 157.635 93.61) (end 162.4343 98.4093) (width 0.2) (layer "F.Cu") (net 14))
 (segment (start 162.4343 98.4093) (end 183.1257 98.4093) (width 0.2) (layer "F.Cu") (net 14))
 (via (at 183.1257 98.4093) (size 0.6) (drill 0.3) (layers "F.Cu" "B.Cu") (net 14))
 (segment (start 188.4315 121.5783) (end 188.7 121.5783) (width 0.2) (layer "B.Cu") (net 14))
 (segment (start 183.1257 116.2725) (end 188.4315 121.5783) (width 0.2) (layer "B.Cu") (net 14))
 (segment (start 183.1257 98.4093) (end 183.1257 116.2725) (width 0.2) (layer "B.Cu") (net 14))
 (segment (start 188.7 122.73) (end 188.7 121.5783) (width 0.2) (layer "B.Cu") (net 14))
 (segment (start 131.155 92.03) (end 134.475 88.71) (width 0.2) (layer "F.Cu") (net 20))
 (segment (start 131.155 93.61) (end 131.155 92.03) (width 0.2) (layer "F.Cu") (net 20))
 (segment (start 137.775 93.61) (end 137.775 92.03) (width 0.2) (layer "F.Cu") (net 4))
 (segment (start 137.775 92.03) (end 141.095 88.71) (width 0.2) (layer "F.Cu") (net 4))
 (segment (start 147.715 90.29) (end 144.395 93.61) (width 0.2) (layer "F.Cu") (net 2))
 (segment (start 147.715 88.71) (end 147.715 90.29) (width 0.2) (layer "F.Cu") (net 2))
 (segment (start 151.015 92.03) (end 154.335 88.71) (width 0.2) (layer "F.Cu") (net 15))
 (segment (start 151.015 93.61) (end 151.015 92.03) (width 0.2) (layer "F.Cu") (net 15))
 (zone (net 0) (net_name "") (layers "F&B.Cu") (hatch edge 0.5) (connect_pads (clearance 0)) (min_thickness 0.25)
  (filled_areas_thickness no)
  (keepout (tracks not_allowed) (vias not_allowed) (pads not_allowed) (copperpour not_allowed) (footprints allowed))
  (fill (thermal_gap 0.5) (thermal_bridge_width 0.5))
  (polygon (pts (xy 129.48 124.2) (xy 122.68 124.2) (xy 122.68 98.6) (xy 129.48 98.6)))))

